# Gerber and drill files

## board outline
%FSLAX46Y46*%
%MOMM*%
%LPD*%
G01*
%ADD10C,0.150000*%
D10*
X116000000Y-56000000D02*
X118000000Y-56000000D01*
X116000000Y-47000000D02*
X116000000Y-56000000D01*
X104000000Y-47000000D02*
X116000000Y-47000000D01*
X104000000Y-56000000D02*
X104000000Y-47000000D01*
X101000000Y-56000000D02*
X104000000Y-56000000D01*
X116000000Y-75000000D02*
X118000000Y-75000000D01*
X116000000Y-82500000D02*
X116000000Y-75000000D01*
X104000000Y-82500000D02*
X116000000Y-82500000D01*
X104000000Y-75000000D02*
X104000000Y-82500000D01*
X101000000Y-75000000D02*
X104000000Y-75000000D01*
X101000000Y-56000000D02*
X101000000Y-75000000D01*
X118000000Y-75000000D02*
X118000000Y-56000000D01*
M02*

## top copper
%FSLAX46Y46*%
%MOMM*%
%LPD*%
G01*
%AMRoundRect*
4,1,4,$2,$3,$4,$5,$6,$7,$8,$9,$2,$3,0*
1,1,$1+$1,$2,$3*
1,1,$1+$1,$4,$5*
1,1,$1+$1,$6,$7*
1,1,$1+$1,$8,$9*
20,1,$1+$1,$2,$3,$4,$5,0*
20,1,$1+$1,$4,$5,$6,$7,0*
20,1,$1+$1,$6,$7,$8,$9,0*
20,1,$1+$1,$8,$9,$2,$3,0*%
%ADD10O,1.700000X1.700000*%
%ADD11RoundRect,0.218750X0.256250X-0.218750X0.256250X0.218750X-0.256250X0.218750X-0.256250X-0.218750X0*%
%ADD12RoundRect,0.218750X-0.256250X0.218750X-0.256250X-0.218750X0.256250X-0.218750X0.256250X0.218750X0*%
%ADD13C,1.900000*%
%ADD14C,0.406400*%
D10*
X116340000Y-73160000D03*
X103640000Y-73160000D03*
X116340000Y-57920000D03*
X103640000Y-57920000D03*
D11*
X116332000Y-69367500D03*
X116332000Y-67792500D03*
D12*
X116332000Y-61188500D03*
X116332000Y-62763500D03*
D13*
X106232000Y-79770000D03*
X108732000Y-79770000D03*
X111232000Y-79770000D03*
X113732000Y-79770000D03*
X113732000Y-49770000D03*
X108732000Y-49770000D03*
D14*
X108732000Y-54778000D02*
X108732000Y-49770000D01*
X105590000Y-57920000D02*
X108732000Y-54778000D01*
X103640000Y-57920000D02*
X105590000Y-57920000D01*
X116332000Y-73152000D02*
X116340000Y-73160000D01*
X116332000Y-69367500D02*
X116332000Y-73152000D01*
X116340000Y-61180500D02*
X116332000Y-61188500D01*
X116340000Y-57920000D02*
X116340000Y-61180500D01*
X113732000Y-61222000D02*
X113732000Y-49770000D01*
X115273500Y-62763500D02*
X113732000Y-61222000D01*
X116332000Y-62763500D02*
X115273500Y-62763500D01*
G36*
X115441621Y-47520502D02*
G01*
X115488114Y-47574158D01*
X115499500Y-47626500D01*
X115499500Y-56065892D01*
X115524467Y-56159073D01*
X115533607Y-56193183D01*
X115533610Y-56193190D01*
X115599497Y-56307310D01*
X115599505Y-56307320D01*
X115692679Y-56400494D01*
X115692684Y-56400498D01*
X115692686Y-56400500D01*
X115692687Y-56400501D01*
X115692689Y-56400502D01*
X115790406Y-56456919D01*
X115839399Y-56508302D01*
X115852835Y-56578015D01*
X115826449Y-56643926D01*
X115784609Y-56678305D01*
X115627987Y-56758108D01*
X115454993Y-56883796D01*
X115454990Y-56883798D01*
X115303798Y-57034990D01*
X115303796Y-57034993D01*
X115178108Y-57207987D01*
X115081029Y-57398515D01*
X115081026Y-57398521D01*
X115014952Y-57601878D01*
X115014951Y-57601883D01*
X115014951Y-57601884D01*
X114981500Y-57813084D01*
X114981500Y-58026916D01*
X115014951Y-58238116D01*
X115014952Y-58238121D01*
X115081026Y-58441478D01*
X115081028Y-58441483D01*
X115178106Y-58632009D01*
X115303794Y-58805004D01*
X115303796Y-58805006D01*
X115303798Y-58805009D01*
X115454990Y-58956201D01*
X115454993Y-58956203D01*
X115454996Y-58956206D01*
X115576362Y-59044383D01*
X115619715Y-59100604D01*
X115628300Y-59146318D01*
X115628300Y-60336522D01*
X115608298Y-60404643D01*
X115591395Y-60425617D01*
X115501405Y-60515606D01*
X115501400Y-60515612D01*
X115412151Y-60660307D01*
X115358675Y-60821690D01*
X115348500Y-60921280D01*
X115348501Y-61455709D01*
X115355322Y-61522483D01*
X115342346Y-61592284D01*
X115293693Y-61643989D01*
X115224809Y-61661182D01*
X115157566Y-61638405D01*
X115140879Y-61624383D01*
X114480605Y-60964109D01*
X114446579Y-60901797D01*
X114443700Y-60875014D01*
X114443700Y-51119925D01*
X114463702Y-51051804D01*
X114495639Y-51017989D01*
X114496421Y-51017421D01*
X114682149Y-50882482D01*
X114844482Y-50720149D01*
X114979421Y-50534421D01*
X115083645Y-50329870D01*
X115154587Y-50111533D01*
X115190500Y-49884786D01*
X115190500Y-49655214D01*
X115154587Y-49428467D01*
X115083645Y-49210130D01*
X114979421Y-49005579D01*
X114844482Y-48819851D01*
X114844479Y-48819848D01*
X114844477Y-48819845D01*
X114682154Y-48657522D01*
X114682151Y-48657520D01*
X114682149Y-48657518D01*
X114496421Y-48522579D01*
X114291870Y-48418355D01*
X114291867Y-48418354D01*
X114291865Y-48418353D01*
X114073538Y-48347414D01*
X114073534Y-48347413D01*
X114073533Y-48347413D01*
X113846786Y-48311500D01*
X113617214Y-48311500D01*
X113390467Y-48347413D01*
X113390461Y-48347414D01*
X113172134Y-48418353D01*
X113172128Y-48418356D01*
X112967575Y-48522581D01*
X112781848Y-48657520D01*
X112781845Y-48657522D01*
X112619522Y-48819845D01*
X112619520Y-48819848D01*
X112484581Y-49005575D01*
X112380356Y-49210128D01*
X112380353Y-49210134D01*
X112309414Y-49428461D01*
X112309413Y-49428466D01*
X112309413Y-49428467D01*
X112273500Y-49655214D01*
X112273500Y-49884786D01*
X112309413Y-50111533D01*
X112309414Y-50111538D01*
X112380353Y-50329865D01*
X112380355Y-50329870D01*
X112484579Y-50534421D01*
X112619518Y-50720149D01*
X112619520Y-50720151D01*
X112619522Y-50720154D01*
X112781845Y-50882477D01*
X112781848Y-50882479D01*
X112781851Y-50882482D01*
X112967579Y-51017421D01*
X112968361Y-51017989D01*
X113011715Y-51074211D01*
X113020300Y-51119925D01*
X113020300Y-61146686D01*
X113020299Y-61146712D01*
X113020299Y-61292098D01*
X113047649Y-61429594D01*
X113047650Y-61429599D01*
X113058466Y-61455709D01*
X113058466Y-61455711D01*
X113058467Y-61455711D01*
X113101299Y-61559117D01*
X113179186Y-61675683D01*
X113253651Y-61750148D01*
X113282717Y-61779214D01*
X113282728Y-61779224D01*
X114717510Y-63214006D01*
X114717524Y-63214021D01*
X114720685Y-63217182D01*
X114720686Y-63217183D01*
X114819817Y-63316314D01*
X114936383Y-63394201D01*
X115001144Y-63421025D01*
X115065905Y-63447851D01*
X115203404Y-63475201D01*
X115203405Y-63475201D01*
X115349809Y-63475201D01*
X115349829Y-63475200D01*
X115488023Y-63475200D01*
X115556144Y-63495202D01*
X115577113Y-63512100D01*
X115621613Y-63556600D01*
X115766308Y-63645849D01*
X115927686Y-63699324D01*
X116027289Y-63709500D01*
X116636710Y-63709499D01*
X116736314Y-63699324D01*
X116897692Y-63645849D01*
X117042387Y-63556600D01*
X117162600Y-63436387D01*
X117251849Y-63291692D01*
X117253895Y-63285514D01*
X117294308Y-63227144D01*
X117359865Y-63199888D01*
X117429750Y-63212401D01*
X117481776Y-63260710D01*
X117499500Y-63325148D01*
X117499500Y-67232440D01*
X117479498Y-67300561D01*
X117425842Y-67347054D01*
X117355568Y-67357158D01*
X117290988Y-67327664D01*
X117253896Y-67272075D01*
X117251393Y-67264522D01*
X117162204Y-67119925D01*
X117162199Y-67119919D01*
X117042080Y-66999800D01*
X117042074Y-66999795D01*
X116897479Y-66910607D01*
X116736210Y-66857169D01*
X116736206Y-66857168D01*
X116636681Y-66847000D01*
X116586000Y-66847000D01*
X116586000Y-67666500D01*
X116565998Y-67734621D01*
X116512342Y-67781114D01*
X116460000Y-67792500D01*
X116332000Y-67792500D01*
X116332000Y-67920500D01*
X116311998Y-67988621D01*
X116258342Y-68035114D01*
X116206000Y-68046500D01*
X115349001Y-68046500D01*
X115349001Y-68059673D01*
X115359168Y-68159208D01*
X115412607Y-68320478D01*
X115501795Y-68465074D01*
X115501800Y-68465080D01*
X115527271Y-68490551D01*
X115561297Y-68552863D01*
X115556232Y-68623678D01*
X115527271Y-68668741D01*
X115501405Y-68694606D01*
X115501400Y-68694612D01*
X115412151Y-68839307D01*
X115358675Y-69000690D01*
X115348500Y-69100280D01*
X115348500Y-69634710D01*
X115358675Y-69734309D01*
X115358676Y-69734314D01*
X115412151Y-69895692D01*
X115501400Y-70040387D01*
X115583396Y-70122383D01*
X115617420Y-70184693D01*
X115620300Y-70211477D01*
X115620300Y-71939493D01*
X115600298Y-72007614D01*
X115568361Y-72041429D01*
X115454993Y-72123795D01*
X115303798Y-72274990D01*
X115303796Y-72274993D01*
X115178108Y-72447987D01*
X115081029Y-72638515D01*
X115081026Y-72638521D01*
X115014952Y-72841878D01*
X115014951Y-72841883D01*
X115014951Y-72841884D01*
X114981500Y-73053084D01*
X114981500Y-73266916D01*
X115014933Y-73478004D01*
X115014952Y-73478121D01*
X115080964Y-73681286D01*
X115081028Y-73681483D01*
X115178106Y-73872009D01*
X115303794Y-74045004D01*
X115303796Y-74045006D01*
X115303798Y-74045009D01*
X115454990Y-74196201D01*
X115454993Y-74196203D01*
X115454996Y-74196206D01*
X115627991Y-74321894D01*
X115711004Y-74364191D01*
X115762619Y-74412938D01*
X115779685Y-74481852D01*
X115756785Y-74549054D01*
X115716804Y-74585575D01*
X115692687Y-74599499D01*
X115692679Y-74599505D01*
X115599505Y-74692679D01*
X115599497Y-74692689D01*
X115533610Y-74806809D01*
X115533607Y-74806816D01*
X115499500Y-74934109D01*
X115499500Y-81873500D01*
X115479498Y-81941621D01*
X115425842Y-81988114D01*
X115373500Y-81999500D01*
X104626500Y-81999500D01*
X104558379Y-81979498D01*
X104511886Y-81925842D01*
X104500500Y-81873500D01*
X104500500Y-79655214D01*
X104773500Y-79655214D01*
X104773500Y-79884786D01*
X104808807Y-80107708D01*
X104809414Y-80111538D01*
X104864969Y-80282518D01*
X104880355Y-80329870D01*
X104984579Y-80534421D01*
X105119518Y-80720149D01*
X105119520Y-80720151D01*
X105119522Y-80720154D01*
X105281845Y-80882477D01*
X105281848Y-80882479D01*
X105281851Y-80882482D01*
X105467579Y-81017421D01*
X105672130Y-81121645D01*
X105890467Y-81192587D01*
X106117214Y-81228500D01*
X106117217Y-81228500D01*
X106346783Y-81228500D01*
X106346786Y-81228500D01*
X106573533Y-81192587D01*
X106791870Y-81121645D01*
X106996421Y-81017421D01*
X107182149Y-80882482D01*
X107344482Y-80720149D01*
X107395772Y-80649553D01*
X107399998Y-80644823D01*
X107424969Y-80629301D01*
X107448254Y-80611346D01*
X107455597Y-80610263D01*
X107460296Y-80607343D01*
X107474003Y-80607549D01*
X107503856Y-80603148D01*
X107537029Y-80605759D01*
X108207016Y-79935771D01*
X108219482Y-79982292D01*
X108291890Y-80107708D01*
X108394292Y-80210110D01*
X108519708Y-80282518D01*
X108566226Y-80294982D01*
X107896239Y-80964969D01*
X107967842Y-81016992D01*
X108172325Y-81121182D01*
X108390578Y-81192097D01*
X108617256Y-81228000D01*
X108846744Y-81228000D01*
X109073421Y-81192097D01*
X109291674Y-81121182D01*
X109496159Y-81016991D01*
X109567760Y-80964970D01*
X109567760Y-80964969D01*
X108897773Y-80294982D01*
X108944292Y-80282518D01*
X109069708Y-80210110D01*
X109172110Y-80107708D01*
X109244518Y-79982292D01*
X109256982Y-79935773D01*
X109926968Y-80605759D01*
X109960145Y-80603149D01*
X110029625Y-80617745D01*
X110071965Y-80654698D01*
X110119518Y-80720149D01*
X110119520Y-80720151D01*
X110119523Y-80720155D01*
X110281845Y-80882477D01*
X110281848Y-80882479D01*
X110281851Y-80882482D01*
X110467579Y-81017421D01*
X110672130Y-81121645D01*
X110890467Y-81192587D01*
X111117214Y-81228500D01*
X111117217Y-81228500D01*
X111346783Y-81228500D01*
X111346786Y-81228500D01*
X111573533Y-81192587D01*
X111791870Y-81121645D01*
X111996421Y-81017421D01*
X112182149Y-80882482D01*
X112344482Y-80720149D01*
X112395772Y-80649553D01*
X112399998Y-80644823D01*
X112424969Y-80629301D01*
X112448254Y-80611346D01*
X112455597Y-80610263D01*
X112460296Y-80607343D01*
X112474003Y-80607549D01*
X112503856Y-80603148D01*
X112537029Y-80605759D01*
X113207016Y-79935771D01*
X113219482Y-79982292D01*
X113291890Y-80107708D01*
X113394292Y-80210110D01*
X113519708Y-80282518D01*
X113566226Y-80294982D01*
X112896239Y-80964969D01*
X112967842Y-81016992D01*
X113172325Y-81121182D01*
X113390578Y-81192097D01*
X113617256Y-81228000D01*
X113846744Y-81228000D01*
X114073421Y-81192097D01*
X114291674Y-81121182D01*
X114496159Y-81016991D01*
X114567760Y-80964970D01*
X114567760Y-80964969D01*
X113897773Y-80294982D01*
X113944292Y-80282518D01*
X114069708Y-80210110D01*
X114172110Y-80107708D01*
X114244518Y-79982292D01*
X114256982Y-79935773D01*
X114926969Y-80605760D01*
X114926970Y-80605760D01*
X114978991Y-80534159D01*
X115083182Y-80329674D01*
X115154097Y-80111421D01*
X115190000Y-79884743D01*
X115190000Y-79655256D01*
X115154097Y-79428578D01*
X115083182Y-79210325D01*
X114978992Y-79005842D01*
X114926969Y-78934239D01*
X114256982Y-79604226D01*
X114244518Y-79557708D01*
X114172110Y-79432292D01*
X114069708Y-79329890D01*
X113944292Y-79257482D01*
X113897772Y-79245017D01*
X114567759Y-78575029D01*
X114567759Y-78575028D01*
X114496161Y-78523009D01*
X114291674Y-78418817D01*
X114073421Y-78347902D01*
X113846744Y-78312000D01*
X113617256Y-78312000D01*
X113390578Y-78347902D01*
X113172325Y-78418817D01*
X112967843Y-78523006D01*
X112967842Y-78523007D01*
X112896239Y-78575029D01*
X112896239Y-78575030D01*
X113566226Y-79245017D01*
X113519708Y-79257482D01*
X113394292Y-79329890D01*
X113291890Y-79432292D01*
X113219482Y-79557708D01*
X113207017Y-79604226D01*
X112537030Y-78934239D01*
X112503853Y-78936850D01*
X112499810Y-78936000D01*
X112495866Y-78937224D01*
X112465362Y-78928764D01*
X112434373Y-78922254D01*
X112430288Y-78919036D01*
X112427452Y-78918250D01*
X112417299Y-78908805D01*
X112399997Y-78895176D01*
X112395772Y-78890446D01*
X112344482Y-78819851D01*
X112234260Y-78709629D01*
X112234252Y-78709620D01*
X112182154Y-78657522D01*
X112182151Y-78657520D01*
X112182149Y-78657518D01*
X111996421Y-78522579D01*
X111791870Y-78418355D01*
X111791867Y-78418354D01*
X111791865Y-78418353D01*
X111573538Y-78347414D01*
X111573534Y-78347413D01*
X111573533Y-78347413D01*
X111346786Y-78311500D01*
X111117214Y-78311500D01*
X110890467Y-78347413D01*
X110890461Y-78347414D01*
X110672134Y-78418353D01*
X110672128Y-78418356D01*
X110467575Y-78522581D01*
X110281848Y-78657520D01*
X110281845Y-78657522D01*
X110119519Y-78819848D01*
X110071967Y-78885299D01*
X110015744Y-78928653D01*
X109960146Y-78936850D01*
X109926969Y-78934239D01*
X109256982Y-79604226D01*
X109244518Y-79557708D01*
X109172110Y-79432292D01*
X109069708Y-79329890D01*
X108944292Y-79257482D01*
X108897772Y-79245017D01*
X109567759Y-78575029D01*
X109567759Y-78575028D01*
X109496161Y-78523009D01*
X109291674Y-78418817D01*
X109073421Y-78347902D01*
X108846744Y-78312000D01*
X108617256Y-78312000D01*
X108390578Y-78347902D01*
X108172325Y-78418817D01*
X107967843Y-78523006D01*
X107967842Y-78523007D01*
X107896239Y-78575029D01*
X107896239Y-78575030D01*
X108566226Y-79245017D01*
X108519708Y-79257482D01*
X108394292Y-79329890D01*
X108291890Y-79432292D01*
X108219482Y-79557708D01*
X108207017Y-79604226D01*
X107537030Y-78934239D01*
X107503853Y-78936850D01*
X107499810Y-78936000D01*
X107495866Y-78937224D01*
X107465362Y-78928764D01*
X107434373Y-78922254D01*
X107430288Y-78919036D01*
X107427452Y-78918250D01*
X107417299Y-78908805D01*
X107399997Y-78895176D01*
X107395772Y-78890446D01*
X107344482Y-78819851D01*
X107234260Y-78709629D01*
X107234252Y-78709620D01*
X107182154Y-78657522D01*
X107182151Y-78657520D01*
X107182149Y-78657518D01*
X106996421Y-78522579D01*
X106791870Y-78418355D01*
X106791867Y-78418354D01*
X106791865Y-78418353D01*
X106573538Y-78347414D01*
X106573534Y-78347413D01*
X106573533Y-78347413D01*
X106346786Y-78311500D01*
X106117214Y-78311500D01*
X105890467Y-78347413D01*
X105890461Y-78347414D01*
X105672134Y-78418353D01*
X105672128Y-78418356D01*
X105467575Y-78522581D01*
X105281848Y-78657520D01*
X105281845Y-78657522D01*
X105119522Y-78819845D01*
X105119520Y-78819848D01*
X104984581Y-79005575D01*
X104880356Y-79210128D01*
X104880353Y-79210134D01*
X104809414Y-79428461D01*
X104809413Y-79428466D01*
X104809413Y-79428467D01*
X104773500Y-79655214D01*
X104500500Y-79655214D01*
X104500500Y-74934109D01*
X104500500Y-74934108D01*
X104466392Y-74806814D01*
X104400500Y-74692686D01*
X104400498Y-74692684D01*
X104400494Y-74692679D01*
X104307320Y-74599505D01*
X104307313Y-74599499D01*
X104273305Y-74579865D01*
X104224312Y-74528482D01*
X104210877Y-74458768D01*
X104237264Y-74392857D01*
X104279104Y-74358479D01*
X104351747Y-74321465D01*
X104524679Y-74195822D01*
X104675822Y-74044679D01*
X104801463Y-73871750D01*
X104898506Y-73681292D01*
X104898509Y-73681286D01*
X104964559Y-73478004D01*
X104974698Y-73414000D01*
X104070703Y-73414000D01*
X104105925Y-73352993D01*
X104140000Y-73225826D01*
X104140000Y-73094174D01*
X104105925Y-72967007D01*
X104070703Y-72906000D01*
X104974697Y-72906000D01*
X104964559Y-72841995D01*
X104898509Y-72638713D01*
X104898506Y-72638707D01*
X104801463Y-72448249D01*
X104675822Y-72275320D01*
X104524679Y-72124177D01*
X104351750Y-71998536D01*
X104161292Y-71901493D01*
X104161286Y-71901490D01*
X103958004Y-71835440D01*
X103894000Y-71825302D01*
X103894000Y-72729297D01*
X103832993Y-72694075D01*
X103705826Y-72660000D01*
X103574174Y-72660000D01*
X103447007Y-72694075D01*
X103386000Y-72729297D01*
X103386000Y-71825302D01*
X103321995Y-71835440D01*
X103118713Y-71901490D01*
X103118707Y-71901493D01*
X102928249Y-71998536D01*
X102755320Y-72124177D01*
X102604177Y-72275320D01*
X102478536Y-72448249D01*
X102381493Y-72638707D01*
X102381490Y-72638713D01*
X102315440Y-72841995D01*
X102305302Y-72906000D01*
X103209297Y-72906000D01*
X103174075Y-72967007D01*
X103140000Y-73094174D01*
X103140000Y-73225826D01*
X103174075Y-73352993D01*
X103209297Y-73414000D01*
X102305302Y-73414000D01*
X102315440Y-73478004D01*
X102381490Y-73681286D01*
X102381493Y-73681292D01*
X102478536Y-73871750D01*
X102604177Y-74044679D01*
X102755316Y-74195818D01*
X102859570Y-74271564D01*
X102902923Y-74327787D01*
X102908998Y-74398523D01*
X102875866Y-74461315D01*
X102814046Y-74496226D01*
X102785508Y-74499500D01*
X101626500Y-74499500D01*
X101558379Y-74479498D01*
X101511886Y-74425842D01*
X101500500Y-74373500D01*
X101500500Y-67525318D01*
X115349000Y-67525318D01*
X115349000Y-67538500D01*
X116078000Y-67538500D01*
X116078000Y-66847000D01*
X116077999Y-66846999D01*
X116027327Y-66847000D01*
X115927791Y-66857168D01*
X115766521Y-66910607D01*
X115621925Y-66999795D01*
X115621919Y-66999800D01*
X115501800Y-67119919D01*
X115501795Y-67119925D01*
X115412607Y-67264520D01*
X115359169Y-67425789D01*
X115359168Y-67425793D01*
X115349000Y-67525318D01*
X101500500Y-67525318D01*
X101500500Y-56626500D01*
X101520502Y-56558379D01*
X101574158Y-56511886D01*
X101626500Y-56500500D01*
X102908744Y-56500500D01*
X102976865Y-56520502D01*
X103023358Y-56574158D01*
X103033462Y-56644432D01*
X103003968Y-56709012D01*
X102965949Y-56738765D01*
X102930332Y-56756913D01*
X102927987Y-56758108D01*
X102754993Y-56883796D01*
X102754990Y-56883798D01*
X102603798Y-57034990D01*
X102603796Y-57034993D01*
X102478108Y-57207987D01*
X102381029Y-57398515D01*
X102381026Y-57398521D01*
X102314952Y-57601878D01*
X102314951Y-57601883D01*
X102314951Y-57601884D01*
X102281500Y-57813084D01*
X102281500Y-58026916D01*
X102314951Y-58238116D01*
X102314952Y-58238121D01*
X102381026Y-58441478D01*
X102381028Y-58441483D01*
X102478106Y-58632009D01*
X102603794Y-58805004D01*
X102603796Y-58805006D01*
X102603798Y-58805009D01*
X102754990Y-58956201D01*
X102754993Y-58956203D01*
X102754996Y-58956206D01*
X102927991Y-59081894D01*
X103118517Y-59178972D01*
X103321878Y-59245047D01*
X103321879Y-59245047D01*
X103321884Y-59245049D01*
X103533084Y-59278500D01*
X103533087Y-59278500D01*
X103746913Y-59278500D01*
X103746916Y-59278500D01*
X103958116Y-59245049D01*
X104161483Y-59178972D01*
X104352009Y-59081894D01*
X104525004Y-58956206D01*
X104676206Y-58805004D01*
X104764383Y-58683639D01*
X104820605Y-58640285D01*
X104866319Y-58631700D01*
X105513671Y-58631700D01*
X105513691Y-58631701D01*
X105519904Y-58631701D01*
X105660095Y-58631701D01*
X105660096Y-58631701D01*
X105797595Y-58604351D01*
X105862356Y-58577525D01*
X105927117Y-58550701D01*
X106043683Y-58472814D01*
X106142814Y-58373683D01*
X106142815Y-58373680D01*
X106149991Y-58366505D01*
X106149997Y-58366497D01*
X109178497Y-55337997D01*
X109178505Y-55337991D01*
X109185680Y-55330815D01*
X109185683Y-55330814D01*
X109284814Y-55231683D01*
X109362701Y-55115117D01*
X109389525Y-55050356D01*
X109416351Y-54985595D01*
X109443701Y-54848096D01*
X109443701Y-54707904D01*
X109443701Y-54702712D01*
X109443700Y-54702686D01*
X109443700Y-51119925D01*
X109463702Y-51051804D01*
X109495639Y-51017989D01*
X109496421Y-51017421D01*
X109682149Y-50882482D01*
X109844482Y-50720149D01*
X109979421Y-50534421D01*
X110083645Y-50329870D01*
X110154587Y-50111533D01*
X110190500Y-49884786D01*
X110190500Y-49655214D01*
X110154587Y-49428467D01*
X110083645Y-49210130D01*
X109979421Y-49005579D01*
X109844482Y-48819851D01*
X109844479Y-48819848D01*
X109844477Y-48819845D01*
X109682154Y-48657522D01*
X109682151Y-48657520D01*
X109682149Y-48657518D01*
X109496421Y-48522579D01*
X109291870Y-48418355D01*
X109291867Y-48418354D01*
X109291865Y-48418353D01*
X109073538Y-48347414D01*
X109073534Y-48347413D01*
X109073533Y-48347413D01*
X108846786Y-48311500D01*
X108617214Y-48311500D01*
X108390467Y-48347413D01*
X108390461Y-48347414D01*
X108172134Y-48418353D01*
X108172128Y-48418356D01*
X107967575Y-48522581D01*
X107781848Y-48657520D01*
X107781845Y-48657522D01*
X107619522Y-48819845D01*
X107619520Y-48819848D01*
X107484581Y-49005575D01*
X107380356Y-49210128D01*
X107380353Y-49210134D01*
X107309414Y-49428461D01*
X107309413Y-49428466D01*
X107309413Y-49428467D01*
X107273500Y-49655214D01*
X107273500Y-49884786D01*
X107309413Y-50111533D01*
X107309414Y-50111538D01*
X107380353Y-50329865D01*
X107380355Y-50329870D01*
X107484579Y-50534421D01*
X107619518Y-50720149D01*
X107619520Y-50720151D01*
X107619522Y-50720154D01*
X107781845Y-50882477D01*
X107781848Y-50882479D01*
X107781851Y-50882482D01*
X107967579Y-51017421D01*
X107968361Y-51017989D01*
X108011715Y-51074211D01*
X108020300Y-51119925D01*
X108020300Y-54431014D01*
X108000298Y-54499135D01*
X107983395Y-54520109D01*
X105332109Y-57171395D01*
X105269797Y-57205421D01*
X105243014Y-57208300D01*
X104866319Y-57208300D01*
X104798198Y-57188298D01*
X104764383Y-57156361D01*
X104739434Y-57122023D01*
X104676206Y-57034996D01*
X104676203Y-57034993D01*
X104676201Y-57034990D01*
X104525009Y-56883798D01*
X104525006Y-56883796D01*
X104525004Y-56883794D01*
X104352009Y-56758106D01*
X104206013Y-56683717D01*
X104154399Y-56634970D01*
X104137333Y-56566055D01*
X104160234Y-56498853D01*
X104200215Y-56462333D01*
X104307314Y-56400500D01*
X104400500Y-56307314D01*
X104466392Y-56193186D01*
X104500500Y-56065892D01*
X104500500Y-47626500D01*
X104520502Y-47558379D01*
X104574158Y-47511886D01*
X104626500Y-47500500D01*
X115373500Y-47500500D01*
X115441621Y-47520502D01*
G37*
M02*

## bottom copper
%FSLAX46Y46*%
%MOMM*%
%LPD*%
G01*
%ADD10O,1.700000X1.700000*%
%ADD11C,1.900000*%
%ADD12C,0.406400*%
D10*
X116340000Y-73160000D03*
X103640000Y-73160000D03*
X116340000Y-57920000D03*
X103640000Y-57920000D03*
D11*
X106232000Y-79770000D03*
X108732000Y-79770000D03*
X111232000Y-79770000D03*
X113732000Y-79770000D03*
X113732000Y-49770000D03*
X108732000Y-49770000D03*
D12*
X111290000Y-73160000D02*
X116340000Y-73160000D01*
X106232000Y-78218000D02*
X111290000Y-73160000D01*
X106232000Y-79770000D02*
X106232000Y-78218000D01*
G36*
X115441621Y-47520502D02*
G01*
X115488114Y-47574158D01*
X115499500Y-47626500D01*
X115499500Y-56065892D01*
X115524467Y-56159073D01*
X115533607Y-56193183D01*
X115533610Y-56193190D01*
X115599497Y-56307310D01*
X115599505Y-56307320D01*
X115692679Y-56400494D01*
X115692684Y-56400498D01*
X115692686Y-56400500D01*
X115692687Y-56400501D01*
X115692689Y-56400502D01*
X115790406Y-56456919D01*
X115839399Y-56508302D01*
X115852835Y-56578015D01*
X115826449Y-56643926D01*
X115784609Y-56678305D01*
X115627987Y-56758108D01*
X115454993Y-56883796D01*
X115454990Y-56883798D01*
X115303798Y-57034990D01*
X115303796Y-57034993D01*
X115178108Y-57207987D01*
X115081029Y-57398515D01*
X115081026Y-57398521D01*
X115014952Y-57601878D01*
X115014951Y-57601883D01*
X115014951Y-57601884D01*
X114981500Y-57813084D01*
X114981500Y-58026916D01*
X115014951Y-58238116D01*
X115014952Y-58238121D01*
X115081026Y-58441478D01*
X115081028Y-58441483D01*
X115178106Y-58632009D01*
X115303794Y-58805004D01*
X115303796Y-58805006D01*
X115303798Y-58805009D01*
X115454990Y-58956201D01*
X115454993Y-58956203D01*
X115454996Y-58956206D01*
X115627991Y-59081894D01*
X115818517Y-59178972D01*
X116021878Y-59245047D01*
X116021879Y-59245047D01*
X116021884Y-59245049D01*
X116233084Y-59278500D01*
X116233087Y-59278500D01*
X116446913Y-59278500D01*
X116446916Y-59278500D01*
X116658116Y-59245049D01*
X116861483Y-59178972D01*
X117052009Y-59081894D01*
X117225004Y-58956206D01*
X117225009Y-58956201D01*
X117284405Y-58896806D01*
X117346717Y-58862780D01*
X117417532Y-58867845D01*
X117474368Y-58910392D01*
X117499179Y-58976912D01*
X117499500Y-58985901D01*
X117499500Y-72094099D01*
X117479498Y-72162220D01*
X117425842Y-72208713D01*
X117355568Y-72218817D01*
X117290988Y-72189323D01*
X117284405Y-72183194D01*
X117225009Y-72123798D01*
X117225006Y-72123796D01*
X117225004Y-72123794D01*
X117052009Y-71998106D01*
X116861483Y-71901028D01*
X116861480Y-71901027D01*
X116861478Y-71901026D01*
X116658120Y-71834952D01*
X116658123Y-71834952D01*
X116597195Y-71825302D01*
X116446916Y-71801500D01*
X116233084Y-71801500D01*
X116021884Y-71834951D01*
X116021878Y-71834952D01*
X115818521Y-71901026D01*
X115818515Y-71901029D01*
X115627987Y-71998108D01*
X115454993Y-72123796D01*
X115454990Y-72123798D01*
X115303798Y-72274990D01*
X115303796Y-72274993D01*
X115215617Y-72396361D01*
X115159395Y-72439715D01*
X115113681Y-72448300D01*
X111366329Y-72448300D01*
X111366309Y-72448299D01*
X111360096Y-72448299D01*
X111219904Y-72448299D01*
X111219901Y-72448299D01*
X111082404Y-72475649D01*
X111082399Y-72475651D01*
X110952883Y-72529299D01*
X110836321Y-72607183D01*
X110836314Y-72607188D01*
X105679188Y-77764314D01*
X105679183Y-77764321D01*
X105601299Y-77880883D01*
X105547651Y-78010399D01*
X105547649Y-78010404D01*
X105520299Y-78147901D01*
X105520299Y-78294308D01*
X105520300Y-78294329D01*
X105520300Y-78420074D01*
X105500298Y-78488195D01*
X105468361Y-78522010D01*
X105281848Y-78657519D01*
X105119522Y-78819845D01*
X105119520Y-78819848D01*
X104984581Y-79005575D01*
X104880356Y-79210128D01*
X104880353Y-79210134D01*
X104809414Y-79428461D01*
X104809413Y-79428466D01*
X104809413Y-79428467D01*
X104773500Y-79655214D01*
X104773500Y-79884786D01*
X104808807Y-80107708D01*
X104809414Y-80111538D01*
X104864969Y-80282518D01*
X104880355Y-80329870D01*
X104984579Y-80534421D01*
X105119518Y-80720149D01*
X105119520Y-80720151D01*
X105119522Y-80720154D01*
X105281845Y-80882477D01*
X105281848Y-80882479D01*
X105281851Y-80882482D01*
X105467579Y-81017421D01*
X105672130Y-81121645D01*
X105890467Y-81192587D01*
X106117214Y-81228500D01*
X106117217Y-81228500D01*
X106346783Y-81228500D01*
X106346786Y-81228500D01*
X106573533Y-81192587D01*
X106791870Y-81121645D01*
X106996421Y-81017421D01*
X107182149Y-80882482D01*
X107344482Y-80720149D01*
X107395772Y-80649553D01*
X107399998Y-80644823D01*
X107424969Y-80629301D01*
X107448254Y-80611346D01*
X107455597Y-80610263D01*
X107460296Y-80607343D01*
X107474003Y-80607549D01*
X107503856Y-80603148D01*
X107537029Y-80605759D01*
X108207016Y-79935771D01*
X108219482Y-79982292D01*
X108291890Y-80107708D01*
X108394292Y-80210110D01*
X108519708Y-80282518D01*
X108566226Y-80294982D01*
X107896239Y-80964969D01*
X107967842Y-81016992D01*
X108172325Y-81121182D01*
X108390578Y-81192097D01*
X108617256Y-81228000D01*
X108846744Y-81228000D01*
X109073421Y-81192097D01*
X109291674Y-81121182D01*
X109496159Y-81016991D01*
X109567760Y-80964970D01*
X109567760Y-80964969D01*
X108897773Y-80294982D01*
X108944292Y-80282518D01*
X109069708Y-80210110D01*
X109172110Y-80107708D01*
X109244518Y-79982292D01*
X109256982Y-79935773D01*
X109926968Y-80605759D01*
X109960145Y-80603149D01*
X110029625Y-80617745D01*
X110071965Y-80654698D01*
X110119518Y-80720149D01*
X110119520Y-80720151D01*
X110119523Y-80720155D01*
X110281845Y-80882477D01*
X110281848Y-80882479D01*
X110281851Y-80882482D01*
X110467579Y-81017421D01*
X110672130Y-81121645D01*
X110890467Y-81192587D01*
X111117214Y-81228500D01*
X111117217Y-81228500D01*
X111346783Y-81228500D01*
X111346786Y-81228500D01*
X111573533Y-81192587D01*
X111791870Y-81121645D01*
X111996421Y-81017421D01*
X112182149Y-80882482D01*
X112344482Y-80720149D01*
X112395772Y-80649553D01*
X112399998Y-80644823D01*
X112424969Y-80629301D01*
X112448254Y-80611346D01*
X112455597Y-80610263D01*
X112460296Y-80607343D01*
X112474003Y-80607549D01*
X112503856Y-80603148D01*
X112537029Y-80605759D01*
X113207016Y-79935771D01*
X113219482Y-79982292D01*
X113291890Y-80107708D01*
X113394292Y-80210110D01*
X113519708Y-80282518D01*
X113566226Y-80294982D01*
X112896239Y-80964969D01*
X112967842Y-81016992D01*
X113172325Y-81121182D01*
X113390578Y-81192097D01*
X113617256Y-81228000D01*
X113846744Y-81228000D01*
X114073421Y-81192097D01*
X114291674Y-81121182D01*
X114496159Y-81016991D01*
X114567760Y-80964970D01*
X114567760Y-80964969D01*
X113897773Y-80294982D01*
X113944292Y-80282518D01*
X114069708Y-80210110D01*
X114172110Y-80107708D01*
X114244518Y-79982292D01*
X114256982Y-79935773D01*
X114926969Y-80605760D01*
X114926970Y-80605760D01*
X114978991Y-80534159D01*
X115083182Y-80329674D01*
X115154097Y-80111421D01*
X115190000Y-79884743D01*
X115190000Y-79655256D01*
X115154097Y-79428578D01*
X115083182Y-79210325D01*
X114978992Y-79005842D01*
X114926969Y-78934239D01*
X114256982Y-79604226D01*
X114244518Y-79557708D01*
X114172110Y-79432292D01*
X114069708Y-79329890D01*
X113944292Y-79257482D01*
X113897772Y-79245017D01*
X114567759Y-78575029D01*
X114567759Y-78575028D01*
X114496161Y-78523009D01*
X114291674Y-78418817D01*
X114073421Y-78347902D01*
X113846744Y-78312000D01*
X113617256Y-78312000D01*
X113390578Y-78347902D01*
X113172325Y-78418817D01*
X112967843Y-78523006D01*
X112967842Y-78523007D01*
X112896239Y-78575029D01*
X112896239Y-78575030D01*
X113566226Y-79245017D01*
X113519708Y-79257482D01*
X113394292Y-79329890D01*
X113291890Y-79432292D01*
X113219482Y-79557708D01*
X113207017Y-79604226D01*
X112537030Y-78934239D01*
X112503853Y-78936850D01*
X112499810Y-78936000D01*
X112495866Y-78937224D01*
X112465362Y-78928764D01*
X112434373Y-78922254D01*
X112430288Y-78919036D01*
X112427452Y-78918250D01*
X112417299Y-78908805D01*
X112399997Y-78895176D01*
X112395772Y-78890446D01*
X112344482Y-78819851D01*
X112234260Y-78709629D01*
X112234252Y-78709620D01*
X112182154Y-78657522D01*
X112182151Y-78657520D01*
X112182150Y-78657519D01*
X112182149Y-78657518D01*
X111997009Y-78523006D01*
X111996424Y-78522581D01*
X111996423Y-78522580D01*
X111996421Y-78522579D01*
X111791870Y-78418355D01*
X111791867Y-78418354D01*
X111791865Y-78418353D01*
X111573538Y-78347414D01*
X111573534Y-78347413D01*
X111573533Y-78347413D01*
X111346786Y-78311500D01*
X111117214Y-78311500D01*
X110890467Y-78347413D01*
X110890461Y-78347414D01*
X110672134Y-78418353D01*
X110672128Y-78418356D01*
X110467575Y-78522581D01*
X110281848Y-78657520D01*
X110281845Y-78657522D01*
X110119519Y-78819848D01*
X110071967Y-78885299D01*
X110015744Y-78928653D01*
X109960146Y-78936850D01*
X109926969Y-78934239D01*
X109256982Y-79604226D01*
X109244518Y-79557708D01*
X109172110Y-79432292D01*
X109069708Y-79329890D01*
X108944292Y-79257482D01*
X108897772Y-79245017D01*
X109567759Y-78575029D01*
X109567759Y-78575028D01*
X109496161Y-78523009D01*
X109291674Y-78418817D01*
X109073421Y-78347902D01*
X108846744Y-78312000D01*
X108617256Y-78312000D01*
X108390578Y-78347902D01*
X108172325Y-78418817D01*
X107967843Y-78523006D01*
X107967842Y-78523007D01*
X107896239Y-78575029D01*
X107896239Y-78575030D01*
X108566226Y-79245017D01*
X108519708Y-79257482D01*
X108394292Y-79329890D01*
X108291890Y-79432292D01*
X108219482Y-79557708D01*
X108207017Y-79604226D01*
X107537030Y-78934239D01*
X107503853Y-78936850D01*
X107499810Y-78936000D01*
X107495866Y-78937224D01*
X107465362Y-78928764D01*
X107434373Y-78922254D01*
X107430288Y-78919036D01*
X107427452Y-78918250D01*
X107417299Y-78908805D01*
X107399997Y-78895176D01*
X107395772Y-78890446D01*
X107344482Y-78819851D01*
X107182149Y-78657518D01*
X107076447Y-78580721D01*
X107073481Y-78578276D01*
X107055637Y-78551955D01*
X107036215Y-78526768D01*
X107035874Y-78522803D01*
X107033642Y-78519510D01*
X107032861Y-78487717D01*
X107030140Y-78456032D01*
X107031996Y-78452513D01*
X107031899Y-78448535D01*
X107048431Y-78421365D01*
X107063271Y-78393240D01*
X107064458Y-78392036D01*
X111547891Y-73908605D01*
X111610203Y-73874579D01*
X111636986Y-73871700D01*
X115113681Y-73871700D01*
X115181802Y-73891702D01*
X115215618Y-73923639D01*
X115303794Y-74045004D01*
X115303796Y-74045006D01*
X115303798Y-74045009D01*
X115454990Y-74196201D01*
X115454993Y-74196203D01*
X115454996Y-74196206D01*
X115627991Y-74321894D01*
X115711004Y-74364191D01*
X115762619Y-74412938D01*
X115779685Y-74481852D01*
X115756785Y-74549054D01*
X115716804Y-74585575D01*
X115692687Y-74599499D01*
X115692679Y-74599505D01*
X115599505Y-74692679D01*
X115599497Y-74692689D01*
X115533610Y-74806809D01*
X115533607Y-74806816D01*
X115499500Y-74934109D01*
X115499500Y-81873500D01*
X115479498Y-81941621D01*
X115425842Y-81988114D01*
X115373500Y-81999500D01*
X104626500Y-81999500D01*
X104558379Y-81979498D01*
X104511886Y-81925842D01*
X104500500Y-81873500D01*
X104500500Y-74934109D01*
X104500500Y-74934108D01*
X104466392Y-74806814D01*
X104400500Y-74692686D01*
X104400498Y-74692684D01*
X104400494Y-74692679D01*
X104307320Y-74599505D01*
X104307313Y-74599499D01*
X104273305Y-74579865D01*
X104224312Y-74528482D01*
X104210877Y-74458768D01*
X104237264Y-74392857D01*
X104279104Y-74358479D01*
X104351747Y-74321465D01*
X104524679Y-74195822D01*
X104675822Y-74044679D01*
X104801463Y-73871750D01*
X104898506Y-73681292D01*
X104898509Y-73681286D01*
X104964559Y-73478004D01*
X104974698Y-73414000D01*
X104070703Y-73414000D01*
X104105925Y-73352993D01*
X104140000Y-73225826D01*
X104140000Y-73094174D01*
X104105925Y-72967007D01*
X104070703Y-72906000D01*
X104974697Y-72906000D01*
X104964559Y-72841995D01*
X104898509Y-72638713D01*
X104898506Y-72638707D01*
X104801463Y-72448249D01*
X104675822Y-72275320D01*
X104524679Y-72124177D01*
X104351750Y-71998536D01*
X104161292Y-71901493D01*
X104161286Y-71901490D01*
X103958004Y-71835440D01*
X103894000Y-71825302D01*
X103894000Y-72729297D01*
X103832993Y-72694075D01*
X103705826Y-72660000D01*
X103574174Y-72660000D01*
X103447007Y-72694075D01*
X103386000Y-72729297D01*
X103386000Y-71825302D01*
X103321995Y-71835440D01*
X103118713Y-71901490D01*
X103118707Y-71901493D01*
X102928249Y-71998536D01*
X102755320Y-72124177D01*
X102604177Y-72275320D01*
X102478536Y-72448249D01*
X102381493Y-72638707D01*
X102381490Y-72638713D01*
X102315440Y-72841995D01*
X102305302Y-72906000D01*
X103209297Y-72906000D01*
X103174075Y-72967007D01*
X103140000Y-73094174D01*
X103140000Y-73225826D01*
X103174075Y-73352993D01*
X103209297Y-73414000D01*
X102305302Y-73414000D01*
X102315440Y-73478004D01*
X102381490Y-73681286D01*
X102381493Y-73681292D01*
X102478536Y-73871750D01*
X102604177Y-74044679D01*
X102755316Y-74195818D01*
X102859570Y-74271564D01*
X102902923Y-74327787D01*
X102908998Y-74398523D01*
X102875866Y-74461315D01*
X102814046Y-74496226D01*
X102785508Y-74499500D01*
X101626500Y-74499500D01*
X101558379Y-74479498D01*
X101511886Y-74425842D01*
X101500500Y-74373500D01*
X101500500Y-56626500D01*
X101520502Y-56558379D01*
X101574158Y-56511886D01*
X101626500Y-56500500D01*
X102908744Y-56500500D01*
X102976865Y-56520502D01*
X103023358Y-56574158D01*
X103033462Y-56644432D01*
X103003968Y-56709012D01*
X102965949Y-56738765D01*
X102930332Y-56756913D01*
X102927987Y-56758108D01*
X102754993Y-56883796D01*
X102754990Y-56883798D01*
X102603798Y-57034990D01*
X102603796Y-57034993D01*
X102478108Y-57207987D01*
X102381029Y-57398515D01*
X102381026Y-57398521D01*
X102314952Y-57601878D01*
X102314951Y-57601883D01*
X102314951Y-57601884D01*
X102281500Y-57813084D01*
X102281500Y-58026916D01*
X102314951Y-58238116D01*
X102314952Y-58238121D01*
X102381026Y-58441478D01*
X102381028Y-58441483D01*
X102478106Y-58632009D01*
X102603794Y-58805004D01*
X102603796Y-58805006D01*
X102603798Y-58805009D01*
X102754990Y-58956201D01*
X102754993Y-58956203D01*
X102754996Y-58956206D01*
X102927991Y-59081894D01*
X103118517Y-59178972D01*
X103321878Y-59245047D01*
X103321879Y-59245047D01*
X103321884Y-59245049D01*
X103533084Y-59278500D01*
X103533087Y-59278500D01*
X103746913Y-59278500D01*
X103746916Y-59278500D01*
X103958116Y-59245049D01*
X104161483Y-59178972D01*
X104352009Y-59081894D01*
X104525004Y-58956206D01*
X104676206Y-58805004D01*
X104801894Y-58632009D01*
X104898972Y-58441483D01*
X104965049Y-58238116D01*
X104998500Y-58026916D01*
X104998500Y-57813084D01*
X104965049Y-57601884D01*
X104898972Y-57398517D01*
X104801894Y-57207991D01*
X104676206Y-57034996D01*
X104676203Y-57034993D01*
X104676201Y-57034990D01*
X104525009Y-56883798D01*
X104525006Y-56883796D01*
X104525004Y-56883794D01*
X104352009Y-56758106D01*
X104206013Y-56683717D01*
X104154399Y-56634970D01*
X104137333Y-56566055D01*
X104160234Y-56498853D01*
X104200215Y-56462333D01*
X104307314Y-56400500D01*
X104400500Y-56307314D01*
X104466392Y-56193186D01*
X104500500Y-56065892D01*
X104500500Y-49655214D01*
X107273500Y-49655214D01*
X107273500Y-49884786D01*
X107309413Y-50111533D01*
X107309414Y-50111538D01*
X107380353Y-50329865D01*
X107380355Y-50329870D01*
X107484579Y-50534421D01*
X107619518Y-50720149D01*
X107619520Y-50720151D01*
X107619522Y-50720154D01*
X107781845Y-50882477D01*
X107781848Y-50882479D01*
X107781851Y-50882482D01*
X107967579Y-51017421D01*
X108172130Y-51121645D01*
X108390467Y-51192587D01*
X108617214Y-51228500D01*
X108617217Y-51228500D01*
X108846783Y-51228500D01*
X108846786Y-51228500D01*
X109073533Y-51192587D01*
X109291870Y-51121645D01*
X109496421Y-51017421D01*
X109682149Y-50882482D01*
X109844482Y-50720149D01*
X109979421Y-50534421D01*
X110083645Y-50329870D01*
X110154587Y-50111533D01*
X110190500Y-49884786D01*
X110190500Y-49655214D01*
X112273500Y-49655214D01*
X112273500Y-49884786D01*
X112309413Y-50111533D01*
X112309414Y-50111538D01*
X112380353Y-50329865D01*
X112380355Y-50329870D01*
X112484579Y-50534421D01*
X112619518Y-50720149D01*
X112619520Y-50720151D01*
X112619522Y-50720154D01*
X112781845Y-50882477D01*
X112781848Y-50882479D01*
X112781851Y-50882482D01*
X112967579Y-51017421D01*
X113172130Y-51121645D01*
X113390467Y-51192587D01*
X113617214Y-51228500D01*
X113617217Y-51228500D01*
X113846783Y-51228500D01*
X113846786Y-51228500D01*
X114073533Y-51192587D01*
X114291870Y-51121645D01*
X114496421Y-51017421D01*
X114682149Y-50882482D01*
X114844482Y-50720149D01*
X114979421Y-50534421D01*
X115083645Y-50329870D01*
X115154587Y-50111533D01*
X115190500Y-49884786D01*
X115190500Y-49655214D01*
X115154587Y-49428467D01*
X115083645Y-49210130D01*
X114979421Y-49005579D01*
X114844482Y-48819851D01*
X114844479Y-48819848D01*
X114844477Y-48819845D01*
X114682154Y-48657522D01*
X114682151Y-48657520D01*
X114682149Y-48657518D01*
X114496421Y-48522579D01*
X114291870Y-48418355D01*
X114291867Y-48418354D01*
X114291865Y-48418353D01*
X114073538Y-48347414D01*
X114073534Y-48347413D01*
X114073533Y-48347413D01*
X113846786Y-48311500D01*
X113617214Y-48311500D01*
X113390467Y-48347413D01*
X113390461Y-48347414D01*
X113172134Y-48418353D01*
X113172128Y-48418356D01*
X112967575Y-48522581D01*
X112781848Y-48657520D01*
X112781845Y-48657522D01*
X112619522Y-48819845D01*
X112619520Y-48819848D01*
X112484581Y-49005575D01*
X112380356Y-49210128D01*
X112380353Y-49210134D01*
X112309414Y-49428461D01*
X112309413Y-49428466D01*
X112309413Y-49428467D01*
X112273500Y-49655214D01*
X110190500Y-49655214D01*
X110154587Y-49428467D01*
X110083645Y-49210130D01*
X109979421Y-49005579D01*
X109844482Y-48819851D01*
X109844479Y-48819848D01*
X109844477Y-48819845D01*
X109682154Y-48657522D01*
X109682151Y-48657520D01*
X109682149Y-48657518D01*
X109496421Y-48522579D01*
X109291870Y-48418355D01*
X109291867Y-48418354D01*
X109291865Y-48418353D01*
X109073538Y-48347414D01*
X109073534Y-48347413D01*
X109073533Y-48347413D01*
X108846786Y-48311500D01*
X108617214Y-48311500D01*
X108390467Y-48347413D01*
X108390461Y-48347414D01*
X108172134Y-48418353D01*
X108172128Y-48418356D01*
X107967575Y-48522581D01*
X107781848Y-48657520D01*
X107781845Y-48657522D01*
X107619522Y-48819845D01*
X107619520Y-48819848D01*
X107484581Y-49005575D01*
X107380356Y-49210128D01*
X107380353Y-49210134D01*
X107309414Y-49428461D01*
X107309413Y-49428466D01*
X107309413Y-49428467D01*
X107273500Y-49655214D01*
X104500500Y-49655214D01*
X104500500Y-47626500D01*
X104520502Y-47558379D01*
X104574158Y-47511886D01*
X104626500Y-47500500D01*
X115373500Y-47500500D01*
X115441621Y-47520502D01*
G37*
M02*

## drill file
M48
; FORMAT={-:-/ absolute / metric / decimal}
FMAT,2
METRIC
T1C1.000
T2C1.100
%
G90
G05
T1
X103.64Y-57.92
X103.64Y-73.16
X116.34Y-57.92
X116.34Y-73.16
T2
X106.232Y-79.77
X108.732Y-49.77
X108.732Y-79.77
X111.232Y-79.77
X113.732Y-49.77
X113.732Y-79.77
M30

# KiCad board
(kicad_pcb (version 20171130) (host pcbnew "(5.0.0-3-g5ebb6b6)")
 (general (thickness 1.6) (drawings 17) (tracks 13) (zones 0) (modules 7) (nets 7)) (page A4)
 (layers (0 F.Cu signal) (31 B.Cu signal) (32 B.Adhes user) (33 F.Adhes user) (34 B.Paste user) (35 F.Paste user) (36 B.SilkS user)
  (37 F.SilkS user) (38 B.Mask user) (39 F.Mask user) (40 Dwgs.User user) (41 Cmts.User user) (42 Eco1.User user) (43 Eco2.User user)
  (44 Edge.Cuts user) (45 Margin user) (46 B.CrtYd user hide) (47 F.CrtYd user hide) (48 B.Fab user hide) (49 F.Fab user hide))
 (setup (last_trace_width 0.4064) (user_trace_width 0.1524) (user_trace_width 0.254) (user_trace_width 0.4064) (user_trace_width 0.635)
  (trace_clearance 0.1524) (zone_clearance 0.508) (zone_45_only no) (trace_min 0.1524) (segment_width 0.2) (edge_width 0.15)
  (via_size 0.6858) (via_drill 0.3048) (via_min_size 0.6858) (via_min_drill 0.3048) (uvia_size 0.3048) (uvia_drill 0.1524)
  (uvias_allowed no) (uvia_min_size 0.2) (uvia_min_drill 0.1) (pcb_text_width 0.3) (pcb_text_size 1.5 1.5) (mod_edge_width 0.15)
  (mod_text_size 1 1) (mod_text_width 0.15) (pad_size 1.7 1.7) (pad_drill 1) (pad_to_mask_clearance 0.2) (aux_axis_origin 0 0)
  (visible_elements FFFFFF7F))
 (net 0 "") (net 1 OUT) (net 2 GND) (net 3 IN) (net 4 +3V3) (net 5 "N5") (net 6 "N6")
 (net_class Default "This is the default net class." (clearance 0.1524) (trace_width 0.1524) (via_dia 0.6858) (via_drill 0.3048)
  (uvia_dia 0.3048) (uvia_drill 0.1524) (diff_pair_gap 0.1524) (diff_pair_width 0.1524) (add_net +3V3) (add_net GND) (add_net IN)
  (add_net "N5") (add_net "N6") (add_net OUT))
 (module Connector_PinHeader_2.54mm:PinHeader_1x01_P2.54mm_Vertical (layer B.Cu) (at 116.34 73.16 90)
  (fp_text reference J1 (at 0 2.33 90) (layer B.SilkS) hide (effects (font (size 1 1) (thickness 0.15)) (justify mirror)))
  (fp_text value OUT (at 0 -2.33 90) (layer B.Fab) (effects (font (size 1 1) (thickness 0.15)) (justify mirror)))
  (pad 1 thru_hole oval (at 0 0 90) (size 1.7 1.7) (drill 1) (layers *.Cu *.Mask) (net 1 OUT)))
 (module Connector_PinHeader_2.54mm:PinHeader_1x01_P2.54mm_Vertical (layer B.Cu) (at 103.64 73.16)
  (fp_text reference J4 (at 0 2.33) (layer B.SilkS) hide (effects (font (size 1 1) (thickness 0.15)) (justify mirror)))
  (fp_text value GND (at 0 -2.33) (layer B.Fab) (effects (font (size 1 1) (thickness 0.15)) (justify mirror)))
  (pad 1 thru_hole oval (at 0 0) (size 1.7 1.7) (drill 1) (layers *.Cu *.Mask) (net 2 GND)))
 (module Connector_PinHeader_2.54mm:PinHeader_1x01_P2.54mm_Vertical (layer B.Cu) (at 116.34 57.92 90)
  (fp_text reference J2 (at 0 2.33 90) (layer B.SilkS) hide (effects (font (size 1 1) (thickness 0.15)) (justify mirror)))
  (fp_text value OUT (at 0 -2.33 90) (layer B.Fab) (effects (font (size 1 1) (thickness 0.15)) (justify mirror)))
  (pad 1 thru_hole oval (at 0 0 90) (size 1.7 1.7) (drill 1) (layers *.Cu *.Mask) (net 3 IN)))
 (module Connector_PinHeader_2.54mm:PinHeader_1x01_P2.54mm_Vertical (layer B.Cu) (at 103.64 57.92 270)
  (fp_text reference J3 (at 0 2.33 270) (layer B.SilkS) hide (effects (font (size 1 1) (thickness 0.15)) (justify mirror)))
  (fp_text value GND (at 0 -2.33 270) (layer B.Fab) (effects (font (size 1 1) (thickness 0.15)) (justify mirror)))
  (pad 1 thru_hole oval (at 0 0 270) (size 1.7 1.7) (drill 1) (layers *.Cu *.Mask) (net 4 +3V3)))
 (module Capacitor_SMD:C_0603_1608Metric (layer F.Cu) (at 116.332 68.58 90)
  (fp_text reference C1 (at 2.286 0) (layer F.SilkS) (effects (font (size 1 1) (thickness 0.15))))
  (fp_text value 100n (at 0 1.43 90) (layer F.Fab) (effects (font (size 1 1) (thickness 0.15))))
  (pad 1 smd roundrect (at -0.7875 0 90) (size 0.875 0.95) (layers F.Cu F.Paste F.Mask) (roundrect_rratio 0.25) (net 1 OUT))
  (pad 2 smd roundrect (at 0.7875 0 90) (size 0.875 0.95) (layers F.Cu F.Paste F.Mask) (roundrect_rratio 0.25) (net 2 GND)))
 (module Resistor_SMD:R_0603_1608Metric (layer F.Cu) (at 116.332 61.976 270)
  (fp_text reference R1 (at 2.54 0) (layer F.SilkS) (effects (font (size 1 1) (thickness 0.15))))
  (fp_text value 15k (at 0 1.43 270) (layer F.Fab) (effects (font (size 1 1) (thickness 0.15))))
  (pad 1 smd roundrect (at -0.7875 0 270) (size 0.875 0.95) (layers F.Cu F.Paste F.Mask) (roundrect_rratio 0.25) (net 3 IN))
  (pad 2 smd roundrect (at 0.7875 0 270) (size 0.875 0.95) (layers F.Cu F.Paste F.Mask) (roundrect_rratio 0.25) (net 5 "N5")))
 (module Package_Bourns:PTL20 (layer F.Cu) (at 109.982 64.77 90)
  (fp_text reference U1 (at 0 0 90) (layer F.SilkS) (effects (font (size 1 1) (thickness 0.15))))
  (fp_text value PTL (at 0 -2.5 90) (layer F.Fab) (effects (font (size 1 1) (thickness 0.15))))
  (pad 1 thru_hole circle (at -15 -3.75 90) (size 1.9 1.9) (drill 1.1) (layers *.Cu *.Mask) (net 1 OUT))
  (pad 2 thru_hole circle (at -15 -1.25 90) (size 1.9 1.9) (drill 1.1) (layers *.Cu *.Mask) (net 2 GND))
  (pad 3 thru_hole circle (at -15 1.25 90) (size 1.9 1.9) (drill 1.1) (layers *.Cu *.Mask) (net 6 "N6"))
  (pad 4 thru_hole circle (at -15 3.75 90) (size 1.9 1.9) (drill 1.1) (layers *.Cu *.Mask) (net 2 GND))
  (pad 5 thru_hole circle (at 15 3.75 90) (size 1.9 1.9) (drill 1.1) (layers *.Cu *.Mask) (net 5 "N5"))
  (pad 6 thru_hole circle (at 15 -1.25 90) (size 1.9 1.9) (drill 1.1) (layers *.Cu *.Mask) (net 4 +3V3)))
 (gr_line (start 116 56) (end 118 56) (layer Edge.Cuts) (width 0.15))
 (gr_line (start 116 47) (end 116 56) (layer Edge.Cuts) (width 0.15))
 (gr_line (start 104 47) (end 116 47) (layer Edge.Cuts) (width 0.15))
 (gr_line (start 104 56) (end 104 47) (layer Edge.Cuts) (width 0.15))
 (gr_line (start 101 56) (end 104 56) (layer Edge.Cuts) (width 0.15))
 (gr_line (start 116 75) (end 118 75) (layer Edge.Cuts) (width 0.15))
 (gr_line (start 116 82.5) (end 116 75) (layer Edge.Cuts) (width 0.15))
 (gr_line (start 104 82.5) (end 116 82.5) (layer Edge.Cuts) (width 0.15))
 (gr_line (start 104 75) (end 104 82.5) (layer Edge.Cuts) (width 0.15))
 (gr_line (start 101 75) (end 104 75) (layer Edge.Cuts) (width 0.15))
 (gr_line (start 101 56) (end 101 75) (layer Edge.Cuts) (width 0.15))
 (gr_line (start 118 75) (end 118 56) (layer Edge.Cuts) (width 0.15))
 (segment (start 108.732 54.778) (end 108.732 49.77) (width 0.4064) (layer F.Cu) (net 4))
 (segment (start 105.59 57.92) (end 108.732 54.778) (width 0.4064) (layer F.Cu) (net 4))
 (segment (start 103.64 57.92) (end 105.59 57.92) (width 0.4064) (layer F.Cu) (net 4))
 (segment (start 111.29 73.16) (end 116.34 73.16) (width 0.4064) (layer B.Cu) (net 1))
 (segment (start 106.232 78.218) (end 111.29 73.16) (width 0.4064) (layer B.Cu) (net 1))
 (segment (start 106.232 79.77) (end 106.232 78.218) (width 0.4064) (layer B.Cu) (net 1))
 (segment (start 116.332 73.152) (end 116.34 73.16) (width 0.4064) (layer F.Cu) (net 1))
 (segment (start 116.332 69.3675) (end 116.332 73.152) (width 0.4064) (layer F.Cu) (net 1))
 (segment (start 116.34 61.1805) (end 116.332 61.1885) (width 0.4064) (layer F.Cu) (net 3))
 (segment (start 116.34 57.92) (end 116.34 61.1805) (width 0.4064) (layer F.Cu) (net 3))
 (segment (start 113.732 61.222) (end 113.732 49.77) (width 0.4064) (layer F.Cu) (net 5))
 (segment (start 115.2735 62.7635) (end 113.732 61.222) (width 0.4064) (layer F.Cu) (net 5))
 (segment (start 116.332 62.7635) (end 115.2735 62.7635) (width 0.4064) (layer F.Cu) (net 5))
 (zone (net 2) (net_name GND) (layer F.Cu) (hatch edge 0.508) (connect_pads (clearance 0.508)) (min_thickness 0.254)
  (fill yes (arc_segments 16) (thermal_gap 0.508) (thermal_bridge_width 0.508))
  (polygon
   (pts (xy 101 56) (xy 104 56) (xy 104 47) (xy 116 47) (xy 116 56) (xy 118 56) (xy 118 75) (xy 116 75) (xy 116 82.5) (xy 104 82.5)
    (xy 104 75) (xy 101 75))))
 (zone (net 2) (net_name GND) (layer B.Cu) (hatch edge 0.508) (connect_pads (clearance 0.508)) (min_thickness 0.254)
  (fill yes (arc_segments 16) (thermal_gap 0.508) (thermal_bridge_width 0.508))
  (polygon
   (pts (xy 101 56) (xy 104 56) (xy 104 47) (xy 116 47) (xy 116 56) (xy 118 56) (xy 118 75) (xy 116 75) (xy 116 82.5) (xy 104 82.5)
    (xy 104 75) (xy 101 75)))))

